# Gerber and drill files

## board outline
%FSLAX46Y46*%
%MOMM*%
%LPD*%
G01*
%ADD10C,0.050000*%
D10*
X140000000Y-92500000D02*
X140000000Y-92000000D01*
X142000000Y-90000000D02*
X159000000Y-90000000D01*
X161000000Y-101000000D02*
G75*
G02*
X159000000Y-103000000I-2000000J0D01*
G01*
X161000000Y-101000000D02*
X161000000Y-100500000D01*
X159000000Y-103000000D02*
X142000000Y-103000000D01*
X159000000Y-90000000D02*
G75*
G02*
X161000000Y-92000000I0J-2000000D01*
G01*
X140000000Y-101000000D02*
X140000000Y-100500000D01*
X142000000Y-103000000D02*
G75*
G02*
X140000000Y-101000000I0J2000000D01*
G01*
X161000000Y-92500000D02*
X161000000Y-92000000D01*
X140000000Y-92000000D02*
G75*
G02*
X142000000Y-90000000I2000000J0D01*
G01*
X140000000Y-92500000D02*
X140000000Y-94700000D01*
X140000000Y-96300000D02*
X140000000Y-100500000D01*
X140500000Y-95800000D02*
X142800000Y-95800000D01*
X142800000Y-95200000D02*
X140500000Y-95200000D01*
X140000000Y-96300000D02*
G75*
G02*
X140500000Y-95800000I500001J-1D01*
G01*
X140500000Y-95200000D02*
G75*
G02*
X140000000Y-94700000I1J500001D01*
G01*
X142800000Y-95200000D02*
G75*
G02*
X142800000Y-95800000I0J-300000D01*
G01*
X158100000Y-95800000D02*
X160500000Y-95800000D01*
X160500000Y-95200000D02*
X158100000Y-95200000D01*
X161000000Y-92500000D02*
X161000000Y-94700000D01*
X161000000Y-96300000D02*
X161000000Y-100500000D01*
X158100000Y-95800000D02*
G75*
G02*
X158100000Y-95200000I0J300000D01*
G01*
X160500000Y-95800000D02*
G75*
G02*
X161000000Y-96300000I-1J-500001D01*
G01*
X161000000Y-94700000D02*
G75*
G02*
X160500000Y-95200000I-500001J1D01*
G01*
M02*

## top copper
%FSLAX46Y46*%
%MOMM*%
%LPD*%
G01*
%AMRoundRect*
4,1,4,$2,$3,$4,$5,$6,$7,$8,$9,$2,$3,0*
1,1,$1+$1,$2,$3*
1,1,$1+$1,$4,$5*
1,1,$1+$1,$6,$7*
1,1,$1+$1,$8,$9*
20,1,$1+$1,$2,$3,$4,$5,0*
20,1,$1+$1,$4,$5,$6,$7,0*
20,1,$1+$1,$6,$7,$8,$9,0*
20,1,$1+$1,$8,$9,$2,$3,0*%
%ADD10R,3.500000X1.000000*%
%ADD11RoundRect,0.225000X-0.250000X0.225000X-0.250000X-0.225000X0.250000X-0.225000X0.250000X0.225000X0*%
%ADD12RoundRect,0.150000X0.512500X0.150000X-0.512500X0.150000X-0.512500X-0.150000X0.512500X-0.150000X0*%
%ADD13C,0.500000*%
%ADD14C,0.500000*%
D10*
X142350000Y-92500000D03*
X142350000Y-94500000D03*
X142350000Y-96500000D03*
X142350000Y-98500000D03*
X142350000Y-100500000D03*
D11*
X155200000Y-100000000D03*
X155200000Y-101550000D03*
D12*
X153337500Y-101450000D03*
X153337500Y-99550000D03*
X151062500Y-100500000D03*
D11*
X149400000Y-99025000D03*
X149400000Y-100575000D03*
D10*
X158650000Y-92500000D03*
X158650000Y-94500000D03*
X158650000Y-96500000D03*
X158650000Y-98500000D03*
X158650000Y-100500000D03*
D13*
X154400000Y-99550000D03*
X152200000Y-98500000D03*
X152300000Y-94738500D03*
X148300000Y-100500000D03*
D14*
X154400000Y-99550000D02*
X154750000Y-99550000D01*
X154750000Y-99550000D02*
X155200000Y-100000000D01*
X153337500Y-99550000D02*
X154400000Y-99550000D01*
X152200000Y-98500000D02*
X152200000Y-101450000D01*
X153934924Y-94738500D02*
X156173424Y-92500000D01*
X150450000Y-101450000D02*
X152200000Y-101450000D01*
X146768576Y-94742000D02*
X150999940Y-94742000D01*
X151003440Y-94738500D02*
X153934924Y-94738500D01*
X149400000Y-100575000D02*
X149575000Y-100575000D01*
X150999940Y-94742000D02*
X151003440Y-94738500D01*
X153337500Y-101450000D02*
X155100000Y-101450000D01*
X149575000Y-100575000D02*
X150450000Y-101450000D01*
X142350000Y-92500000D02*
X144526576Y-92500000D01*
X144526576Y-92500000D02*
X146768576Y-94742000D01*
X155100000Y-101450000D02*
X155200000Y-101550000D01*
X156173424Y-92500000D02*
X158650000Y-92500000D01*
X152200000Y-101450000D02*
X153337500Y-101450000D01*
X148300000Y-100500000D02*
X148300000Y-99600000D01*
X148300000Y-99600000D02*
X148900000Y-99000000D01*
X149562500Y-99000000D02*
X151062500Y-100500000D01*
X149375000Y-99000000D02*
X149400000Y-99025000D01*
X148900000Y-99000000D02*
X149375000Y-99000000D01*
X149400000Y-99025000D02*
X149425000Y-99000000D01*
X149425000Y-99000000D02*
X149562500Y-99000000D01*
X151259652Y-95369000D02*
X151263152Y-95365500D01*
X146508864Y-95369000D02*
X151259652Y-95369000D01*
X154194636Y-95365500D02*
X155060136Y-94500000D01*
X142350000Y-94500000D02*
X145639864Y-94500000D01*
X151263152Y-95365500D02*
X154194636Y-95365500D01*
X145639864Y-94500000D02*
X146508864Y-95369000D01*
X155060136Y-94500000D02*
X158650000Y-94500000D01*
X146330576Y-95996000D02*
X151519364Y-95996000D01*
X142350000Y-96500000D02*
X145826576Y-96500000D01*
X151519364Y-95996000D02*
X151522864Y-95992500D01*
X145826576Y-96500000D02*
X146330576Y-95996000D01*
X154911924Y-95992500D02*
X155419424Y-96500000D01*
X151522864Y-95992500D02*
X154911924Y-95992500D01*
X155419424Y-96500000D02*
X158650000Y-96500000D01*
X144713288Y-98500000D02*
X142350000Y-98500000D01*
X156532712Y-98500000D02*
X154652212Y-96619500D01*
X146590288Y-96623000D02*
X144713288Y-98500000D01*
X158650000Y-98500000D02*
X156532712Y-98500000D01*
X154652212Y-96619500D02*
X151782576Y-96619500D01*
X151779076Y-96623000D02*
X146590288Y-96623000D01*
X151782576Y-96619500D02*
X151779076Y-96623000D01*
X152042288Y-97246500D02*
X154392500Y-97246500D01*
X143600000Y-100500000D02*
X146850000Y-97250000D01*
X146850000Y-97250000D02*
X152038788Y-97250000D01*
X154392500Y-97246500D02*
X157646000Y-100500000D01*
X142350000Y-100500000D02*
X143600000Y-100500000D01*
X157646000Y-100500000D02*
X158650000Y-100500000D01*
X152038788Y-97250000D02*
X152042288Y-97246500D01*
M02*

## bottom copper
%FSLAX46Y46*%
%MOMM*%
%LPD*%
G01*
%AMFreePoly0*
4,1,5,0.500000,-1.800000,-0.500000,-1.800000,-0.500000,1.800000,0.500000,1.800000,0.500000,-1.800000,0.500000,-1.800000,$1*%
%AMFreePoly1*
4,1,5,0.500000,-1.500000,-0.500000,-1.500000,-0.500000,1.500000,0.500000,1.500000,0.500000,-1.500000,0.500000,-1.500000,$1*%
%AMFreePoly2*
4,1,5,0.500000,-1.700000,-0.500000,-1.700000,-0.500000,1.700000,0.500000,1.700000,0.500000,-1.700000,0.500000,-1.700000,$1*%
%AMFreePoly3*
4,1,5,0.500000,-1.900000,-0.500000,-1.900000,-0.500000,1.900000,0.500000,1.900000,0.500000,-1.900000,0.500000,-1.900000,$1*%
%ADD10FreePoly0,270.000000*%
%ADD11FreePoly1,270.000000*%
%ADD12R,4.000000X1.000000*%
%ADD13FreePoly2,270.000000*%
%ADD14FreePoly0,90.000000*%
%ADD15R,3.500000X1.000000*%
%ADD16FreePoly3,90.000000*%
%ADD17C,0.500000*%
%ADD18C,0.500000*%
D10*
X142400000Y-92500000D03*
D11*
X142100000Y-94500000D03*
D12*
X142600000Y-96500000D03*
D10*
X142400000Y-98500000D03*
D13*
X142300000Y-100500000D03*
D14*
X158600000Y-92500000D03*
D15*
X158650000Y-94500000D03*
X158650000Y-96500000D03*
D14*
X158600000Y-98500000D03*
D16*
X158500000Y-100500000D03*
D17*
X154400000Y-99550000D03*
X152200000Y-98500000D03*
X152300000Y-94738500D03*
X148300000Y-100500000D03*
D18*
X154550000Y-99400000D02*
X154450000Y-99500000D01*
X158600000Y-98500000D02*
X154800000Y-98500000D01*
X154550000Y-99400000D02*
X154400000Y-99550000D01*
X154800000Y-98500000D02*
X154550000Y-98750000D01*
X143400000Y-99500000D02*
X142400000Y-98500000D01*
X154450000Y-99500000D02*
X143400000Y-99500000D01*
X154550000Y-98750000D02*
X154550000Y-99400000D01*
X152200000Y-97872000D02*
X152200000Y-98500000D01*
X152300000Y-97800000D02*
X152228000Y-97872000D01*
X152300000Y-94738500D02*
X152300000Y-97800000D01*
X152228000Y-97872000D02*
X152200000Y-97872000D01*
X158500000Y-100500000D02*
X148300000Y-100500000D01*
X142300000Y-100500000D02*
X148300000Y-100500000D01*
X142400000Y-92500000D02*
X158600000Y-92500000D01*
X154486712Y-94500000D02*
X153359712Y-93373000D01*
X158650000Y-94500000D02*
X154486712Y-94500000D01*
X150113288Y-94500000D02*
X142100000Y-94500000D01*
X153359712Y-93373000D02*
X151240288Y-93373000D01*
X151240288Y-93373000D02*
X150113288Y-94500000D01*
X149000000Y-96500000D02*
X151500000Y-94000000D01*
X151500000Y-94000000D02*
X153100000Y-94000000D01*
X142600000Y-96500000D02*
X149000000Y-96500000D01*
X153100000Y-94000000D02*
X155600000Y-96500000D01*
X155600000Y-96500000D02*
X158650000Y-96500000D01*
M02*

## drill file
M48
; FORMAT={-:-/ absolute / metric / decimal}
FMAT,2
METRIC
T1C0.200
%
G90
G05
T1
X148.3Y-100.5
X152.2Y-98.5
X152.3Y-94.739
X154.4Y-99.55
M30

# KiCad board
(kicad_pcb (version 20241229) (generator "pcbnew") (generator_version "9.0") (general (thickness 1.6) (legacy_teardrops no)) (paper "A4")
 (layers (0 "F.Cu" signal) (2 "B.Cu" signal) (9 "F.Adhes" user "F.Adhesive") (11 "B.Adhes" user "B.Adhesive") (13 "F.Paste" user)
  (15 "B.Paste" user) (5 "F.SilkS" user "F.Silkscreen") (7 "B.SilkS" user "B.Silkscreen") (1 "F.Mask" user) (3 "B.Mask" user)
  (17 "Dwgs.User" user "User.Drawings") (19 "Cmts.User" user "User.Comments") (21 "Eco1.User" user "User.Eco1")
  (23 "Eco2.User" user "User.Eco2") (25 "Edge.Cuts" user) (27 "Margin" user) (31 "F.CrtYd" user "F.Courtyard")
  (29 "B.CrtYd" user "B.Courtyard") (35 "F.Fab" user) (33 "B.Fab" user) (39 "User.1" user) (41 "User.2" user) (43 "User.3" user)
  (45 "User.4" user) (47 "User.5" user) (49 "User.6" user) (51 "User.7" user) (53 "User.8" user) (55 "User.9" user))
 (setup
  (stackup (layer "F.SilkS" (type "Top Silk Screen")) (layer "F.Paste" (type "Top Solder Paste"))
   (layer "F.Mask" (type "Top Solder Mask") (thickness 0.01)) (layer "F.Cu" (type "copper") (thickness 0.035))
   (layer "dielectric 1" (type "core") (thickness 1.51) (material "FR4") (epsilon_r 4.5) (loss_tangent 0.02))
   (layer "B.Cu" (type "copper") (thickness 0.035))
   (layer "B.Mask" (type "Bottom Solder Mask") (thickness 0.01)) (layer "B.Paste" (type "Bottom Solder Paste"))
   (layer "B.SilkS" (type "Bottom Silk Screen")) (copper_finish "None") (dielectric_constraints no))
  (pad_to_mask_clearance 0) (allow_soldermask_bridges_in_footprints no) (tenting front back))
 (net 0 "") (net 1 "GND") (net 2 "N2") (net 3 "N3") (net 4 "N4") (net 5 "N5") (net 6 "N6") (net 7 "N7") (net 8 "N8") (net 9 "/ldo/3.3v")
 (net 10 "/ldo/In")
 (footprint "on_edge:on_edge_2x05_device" (layer "F.Cu") (at 140 96.5 -90)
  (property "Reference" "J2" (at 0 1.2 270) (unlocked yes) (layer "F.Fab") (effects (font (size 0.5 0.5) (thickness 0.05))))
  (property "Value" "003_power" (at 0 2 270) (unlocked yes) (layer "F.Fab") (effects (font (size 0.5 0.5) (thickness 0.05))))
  (fp_line (start -4 0) (end -1.8 0) (stroke (width 0.05) (type solid)) (layer "Edge.Cuts"))
  (fp_line (start -0.2 0) (end 4 0) (stroke (width 0.05) (type solid)) (layer "Edge.Cuts"))
  (fp_line (start -0.7 -0.5) (end -0.7 -2.8) (stroke (width 0.05) (type solid)) (layer "Edge.Cuts"))
  (fp_line (start -1.3 -2.8) (end -1.3 -0.5) (stroke (width 0.05) (type solid)) (layer "Edge.Cuts"))
  (fp_arc (start -0.2 0) (mid -0.553553 -0.146447) (end -0.7 -0.5) (stroke (width 0.05) (type solid)) (layer "Edge.Cuts"))
  (fp_arc (start -1.3 -0.5) (mid -1.446447 -0.146447) (end -1.8 0) (stroke (width 0.05) (type solid)) (layer "Edge.Cuts"))
  (fp_arc (start -1.3 -2.8) (mid -1 -3.1) (end -0.7 -2.8) (stroke (width 0.05) (type solid)) (layer "Edge.Cuts"))
  (pad "1" smd rect (at -4 -2.35 90) (size 1 3.5) (layers "F.Cu" "F.Mask") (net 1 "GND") (zone_connect 0))
  (pad "2" smd rect (at -2 -2.35 270) (size 1 3.5) (layers "F.Cu" "F.Mask") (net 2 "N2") (zone_connect 0))
  (pad "3" smd rect (at 0 -2.35 270) (size 1 3.5) (layers "F.Cu" "F.Mask") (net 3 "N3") (zone_connect 0))
  (pad "4" smd rect (at 2 -2.35 90) (size 1 3.5) (layers "F.Cu" "F.Mask") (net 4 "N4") (zone_connect 0))
  (pad "5" smd rect (at 4 -2.35 90) (size 1 3.5) (layers "F.Cu" "F.Mask") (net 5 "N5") (zone_connect 0))
  (pad "6" smd custom (at -4 -2.4 270) (size 1 3.6) (layers "B.Cu" "B.Mask") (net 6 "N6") (zone_connect 0)
   (options (clearance outline) (anchor rect)) (primitives))
  (pad "7" smd custom (at -2 -2.1 270) (size 1 3) (layers "B.Cu" "B.Mask") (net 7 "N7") (zone_connect 0)
   (options (clearance outline) (anchor rect)) (primitives))
  (pad "8" smd rect (at 0 -2.6 270) (size 1 4) (layers "B.Cu" "B.Mask") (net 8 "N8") (zone_connect 0))
  (pad "9" smd custom (at 2 -2.4 270) (size 1 3.6) (layers "B.Cu" "B.Mask") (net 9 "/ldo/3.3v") (zone_connect 0)
   (options (clearance outline) (anchor rect)) (primitives))
  (pad "10" smd custom (at 4 -2.3 270) (size 1 3.4) (layers "B.Cu" "B.Mask") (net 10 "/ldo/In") (zone_connect 0)
   (options (clearance outline) (anchor rect)) (primitives))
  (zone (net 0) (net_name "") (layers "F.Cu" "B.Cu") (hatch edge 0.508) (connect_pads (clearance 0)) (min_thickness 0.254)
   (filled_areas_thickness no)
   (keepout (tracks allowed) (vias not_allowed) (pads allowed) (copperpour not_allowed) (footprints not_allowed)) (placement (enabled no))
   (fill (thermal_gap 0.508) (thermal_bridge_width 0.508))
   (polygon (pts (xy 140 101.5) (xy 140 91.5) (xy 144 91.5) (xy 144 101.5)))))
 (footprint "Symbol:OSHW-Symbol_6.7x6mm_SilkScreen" (layer "F.Cu") (at 149.35 94.7)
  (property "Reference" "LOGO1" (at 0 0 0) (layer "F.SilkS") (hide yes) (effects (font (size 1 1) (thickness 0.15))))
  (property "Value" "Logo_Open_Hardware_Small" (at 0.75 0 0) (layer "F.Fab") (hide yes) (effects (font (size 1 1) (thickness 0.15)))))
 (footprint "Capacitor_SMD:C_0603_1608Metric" (layer "F.Cu") (at 155.2 100.775 -90)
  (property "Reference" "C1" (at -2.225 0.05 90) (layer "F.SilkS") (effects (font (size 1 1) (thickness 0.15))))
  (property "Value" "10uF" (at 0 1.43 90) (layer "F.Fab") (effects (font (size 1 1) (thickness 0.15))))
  (pad "1" smd roundrect (at -0.775 0 270) (size 0.9 0.95) (layers "F.Cu" "F.Mask" "F.Paste") (roundrect_rratio 0.25) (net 9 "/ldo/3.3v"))
  (pad "2" smd roundrect (at 0.775 0 270) (size 0.9 0.95) (layers "F.Cu" "F.Mask" "F.Paste") (roundrect_rratio 0.25) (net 1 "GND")))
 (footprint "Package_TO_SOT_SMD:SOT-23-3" (layer "F.Cu") (at 152.2 100.5 180)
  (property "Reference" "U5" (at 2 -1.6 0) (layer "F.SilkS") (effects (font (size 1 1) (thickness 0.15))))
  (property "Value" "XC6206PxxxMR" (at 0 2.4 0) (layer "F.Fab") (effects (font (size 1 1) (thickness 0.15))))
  (pad "1" smd roundrect (at -1.1375 -0.95 180) (size 1.325 0.6) (layers "F.Cu" "F.Mask" "F.Paste") (roundrect_rratio 0.25) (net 1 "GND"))
  (pad "2" smd roundrect (at -1.1375 0.95 180) (size 1.325 0.6) (layers "F.Cu" "F.Mask" "F.Paste") (roundrect_rratio 0.25)
   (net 9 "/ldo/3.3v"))
  (pad "3" smd roundrect (at 1.1375 0 180) (size 1.325 0.6) (layers "F.Cu" "F.Mask" "F.Paste") (roundrect_rratio 0.25) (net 10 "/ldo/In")))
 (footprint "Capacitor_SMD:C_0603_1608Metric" (layer "F.Cu") (at 149.4 99.8 -90)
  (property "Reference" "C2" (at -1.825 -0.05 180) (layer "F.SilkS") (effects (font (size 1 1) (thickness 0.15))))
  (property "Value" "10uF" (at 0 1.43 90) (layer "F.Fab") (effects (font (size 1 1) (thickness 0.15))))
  (pad "1" smd roundrect (at -0.775 0 270) (size 0.9 0.95) (layers "F.Cu" "F.Mask" "F.Paste") (roundrect_rratio 0.25) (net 10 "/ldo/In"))
  (pad "2" smd roundrect (at 0.775 0 270) (size 0.9 0.95) (layers "F.Cu" "F.Mask" "F.Paste") (roundrect_rratio 0.25) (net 1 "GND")))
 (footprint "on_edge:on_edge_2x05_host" (layer "F.Cu") (at 161 96.5 -90)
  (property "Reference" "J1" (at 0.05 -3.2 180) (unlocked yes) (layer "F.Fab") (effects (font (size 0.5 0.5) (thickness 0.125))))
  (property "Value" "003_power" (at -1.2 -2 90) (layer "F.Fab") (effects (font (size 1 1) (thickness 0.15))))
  (fp_line (start -0.7 2.9) (end -0.7 0.5) (stroke (width 0.05) (type solid)) (layer "Edge.Cuts"))
  (fp_line (start -1.3 0.5) (end -1.3 2.9) (stroke (width 0.05) (type solid)) (layer "Edge.Cuts"))
  (fp_line (start -4 0) (end -1.8 0) (stroke (width 0.05) (type solid)) (layer "Edge.Cuts"))
  (fp_line (start -0.2 0) (end 4 0) (stroke (width 0.05) (type solid)) (layer "Edge.Cuts"))
  (fp_arc (start -0.7 2.9) (mid -1 3.2) (end -1.3 2.9) (stroke (width 0.05) (type solid)) (layer "Edge.Cuts"))
  (fp_arc (start -0.7 0.5) (mid -0.553553 0.146447) (end -0.2 0) (stroke (width 0.05) (type solid)) (layer "Edge.Cuts"))
  (fp_arc (start -1.8 0) (mid -1.446447 0.146447) (end -1.3 0.5) (stroke (width 0.05) (type solid)) (layer "Edge.Cuts"))
  (pad "1" smd rect (at -4 2.35 270) (size 1 3.5) (layers "F.Cu" "F.Mask") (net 1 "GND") (zone_connect 0))
  (pad "2" smd rect (at -2 2.35 270) (size 1 3.5) (layers "F.Cu" "F.Mask") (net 2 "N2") (zone_connect 0))
  (pad "3" smd rect (at 0 2.35 270) (size 1 3.5) (layers "F.Cu" "F.Mask") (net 3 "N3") (zone_connect 0))
  (pad "4" smd rect (at 2 2.35 270) (size 1 3.5) (layers "F.Cu" "F.Mask") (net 4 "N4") (zone_connect 0))
  (pad "5" smd rect (at 4 2.35 270) (size 1 3.5) (layers "F.Cu" "F.Mask") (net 5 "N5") (zone_connect 0))
  (pad "6" smd custom (at -4 2.4 90) (size 1 3.6) (layers "B.Cu" "B.Mask") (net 6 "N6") (zone_connect 0)
   (options (clearance outline) (anchor rect)) (primitives))
  (pad "7" smd rect (at -2 2.35 90) (size 1 3.5) (layers "B.Cu" "B.Mask") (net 7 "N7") (zone_connect 0))
  (pad "8" smd rect (at 0 2.35 90) (size 1 3.5) (layers "B.Cu" "B.Mask") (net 8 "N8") (zone_connect 0))
  (pad "9" smd custom (at 2 2.4 90) (size 1 3.6) (layers "B.Cu" "B.Mask") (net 9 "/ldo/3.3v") (zone_connect 0)
   (options (clearance outline) (anchor rect)) (primitives))
  (pad "10" smd custom (at 4 2.5 90) (size 1 3.8) (layers "B.Cu" "B.Mask") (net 10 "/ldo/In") (zone_connect 0)
   (options (clearance outline) (anchor rect)) (primitives))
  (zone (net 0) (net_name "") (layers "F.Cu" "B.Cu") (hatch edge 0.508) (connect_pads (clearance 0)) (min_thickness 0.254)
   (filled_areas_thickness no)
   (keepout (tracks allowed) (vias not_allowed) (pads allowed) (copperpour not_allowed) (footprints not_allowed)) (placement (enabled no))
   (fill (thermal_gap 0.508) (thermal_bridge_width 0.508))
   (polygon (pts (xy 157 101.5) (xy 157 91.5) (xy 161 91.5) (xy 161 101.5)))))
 (gr_line (start 140 92.5) (end 140 92) (stroke (width 0.05) (type solid)) (layer "Edge.Cuts"))
 (gr_line (start 142 90) (end 159 90) (stroke (width 0.05) (type solid)) (layer "Edge.Cuts"))
 (gr_arc (start 161 101) (mid 160.414214 102.414214) (end 159 103) (stroke (width 0.05) (type solid)) (layer "Edge.Cuts"))
 (gr_line (start 161 101) (end 161 100.5) (stroke (width 0.05) (type solid)) (layer "Edge.Cuts"))
 (gr_line (start 159 103) (end 142 103) (stroke (width 0.05) (type solid)) (layer "Edge.Cuts"))
 (gr_arc (start 159 90) (mid 160.414214 90.585786) (end 161 92) (stroke (width 0.05) (type solid)) (layer "Edge.Cuts"))
 (gr_line (start 140 101) (end 140 100.5) (stroke (width 0.05) (type solid)) (layer "Edge.Cuts"))
 (gr_arc (start 142 103) (mid 140.585786 102.414214) (end 140 101) (stroke (width 0.05) (type solid)) (layer "Edge.Cuts"))
 (gr_line (start 161 92.5) (end 161 92) (stroke (width 0.05) (type solid)) (layer "Edge.Cuts"))
 (gr_arc (start 140 92) (mid 140.585786 90.585786) (end 142 90) (stroke (width 0.05) (type solid)) (layer "Edge.Cuts"))
 (segment (start 154.4 99.55) (end 154.75 99.55) (width 0.5) (layer "F.Cu") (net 9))
 (segment (start 154.75 99.55) (end 155.2 100) (width 0.5) (layer "F.Cu") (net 9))
 (segment (start 153.3375 99.55) (end 154.4 99.55) (width 0.5) (layer "F.Cu") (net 9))
 (via (at 154.4 99.55) (size 0.5) (drill 0.2) (layers "F.Cu" "B.Cu") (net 9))
 (segment (start 154.55 99.4) (end 154.45 99.5) (width 0.5) (layer "B.Cu") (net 9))
 (segment (start 158.6 98.5) (end 154.8 98.5) (width 0.5) (layer "B.Cu") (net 9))
 (segment (start 154.55 99.4) (end 154.4 99.55) (width 0.5) (layer "B.Cu") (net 9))
 (segment (start 154.8 98.5) (end 154.55 98.75) (width 0.5) (layer "B.Cu") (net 9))
 (segment (start 143.4 99.5) (end 142.4 98.5) (width 0.5) (layer "B.Cu") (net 9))
 (segment (start 154.45 99.5) (end 143.4 99.5) (width 0.5) (layer "B.Cu") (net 9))
 (segment (start 154.55 98.75) (end 154.55 99.4) (width 0.5) (layer "B.Cu") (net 9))
 (segment (start 152.2 98.5) (end 152.2 101.45) (width 0.5) (layer "F.Cu") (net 1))
 (segment (start 153.934924 94.7385) (end 156.173424 92.5) (width 0.5) (layer "F.Cu") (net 1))
 (segment (start 150.45 101.45) (end 152.2 101.45) (width 0.5) (layer "F.Cu") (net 1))
 (segment (start 146.768576 94.742) (end 150.99994 94.742) (width 0.5) (layer "F.Cu") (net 1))
 (segment (start 151.00344 94.7385) (end 153.934924 94.7385) (width 0.5) (layer "F.Cu") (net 1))
 (segment (start 149.4 100.575) (end 149.575 100.575) (width 0.5) (layer "F.Cu") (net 1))
 (segment (start 150.99994 94.742) (end 151.00344 94.7385) (width 0.5) (layer "F.Cu") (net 1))
 (segment (start 153.3375 101.45) (end 155.1 101.45) (width 0.5) (layer "F.Cu") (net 1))
 (segment (start 149.575 100.575) (end 150.45 101.45) (width 0.5) (layer "F.Cu") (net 1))
 (segment (start 142.35 92.5) (end 144.526576 92.5) (width 0.5) (layer "F.Cu") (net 1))
 (segment (start 144.526576 92.5) (end 146.768576 94.742) (width 0.5) (layer "F.Cu") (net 1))
 (segment (start 155.1 101.45) (end 155.2 101.55) (width 0.5) (layer "F.Cu") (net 1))
 (segment (start 156.173424 92.5) (end 158.65 92.5) (width 0.5) (layer "F.Cu") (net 1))
 (segment (start 152.2 101.45) (end 153.3375 101.45) (width 0.5) (layer "F.Cu") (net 1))
 (via (at 152.2 98.5) (size 0.5) (drill 0.2) (layers "F.Cu" "B.Cu") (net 1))
 (via (at 152.3 94.7385) (size 0.5) (drill 0.2) (layers "F.Cu" "B.Cu") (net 1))
 (segment (start 152.2 97.872) (end 152.2 98.5) (width 0.5) (layer "B.Cu") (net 1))
 (segment (start 152.3 97.8) (end 152.228 97.872) (width 0.5) (layer "B.Cu") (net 1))
 (segment (start 152.3 94.7385) (end 152.3 97.8) (width 0.5) (layer "B.Cu") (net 1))
 (segment (start 152.228 97.872) (end 152.2 97.872) (width 0.5) (layer "B.Cu") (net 1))
 (segment (start 148.3 100.5) (end 148.3 99.6) (width 0.5) (layer "F.Cu") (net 10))
 (segment (start 148.3 99.6) (end 148.9 99) (width 0.5) (layer "F.Cu") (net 10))
 (segment (start 149.5625 99) (end 151.0625 100.5) (width 0.5) (layer "F.Cu") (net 10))
 (segment (start 149.375 99) (end 149.4 99.025) (width 0.5) (layer "F.Cu") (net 10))
 (segment (start 148.9 99) (end 149.375 99) (width 0.5) (layer "F.Cu") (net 10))
 (segment (start 149.4 99.025) (end 149.425 99) (width 0.5) (layer "F.Cu") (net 10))
 (segment (start 149.425 99) (end 149.5625 99) (width 0.5) (layer "F.Cu") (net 10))
 (via (at 148.3 100.5) (size 0.5) (drill 0.2) (layers "F.Cu" "B.Cu") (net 10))
 (segment (start 158.5 100.5) (end 148.3 100.5) (width 0.5) (layer "B.Cu") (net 10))
 (segment (start 142.3 100.5) (end 148.3 100.5) (width 0.5) (layer "B.Cu") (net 10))
 (segment (start 151.259652 95.369) (end 151.263152 95.3655) (width 0.5) (layer "F.Cu") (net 2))
 (segment (start 146.508864 95.369) (end 151.259652 95.369) (width 0.5) (layer "F.Cu") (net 2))
 (segment (start 154.194636 95.3655) (end 155.060136 94.5) (width 0.5) (layer "F.Cu") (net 2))
 (segment (start 142.35 94.5) (end 145.639864 94.5) (width 0.5) (layer "F.Cu") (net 2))
 (segment (start 151.263152 95.3655) (end 154.194636 95.3655) (width 0.5) (layer "F.Cu") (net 2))
 (segment (start 145.639864 94.5) (end 146.508864 95.369) (width 0.5) (layer "F.Cu") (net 2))
 (segment (start 155.060136 94.5) (end 158.65 94.5) (width 0.5) (layer "F.Cu") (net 2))
 (segment (start 146.330576 95.996) (end 151.519364 95.996) (width 0.5) (layer "F.Cu") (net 3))
 (segment (start 142.35 96.5) (end 145.826576 96.5) (width 0.5) (layer "F.Cu") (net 3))
 (segment (start 151.519364 95.996) (end 151.522864 95.9925) (width 0.5) (layer "F.Cu") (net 3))
 (segment (start 145.826576 96.5) (end 146.330576 95.996) (width 0.5) (layer "F.Cu") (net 3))
 (segment (start 154.911924 95.9925) (end 155.419424 96.5) (width 0.5) (layer "F.Cu") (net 3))
 (segment (start 151.522864 95.9925) (end 154.911924 95.9925) (width 0.5) (layer "F.Cu") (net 3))
 (segment (start 155.419424 96.5) (end 158.65 96.5) (width 0.5) (layer "F.Cu") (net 3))
 (segment (start 144.713288 98.5) (end 142.35 98.5) (width 0.5) (layer "F.Cu") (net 4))
 (segment (start 156.532712 98.5) (end 154.652212 96.6195) (width 0.5) (layer "F.Cu") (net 4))
 (segment (start 146.590288 96.623) (end 144.713288 98.5) (width 0.5) (layer "F.Cu") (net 4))
 (segment (start 158.65 98.5) (end 156.532712 98.5) (width 0.5) (layer "F.Cu") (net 4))
 (segment (start 154.652212 96.6195) (end 151.782576 96.6195) (width 0.5) (layer "F.Cu") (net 4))
 (segment (start 151.779076 96.623) (end 146.590288 96.623) (width 0.5) (layer "F.Cu") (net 4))
 (segment (start 151.782576 96.6195) (end 151.779076 96.623) (width 0.5) (layer "F.Cu") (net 4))
 (segment (start 152.042288 97.2465) (end 154.3925 97.2465) (width 0.5) (layer "F.Cu") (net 5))
 (segment (start 143.6 100.5) (end 146.85 97.25) (width 0.5) (layer "F.Cu") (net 5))
 (segment (start 146.85 97.25) (end 152.038788 97.25) (width 0.5) (layer "F.Cu") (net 5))
 (segment (start 154.3925 97.2465) (end 157.646 100.5) (width 0.5) (layer "F.Cu") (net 5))
 (segment (start 142.35 100.5) (end 143.6 100.5) (width 0.5) (layer "F.Cu") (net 5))
 (segment (start 157.646 100.5) (end 158.65 100.5) (width 0.5) (layer "F.Cu") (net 5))
 (segment (start 152.038788 97.25) (end 152.042288 97.2465) (width 0.5) (layer "F.Cu") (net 5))
 (segment (start 142.4 92.5) (end 158.6 92.5) (width 0.5) (layer "B.Cu") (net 6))
 (segment (start 154.486712 94.5) (end 153.359712 93.373) (width 0.5) (layer "B.Cu") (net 7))
 (segment (start 158.65 94.5) (end 154.486712 94.5) (width 0.5) (layer "B.Cu") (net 7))
 (segment (start 150.113288 94.5) (end 142.1 94.5) (width 0.5) (layer "B.Cu") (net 7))
 (segment (start 153.359712 93.373) (end 151.240288 93.373) (width 0.5) (layer "B.Cu") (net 7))
 (segment (start 151.240288 93.373) (end 150.113288 94.5) (width 0.5) (layer "B.Cu") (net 7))
 (segment (start 149 96.5) (end 151.5 94) (width 0.5) (layer "B.Cu") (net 8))
 (segment (start 151.5 94) (end 153.1 94) (width 0.5) (layer "B.Cu") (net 8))
 (segment (start 142.6 96.5) (end 149 96.5) (width 0.5) (layer "B.Cu") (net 8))
 (segment (start 153.1 94) (end 155.6 96.5) (width 0.5) (layer "B.Cu") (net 8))
 (segment (start 155.6 96.5) (end 158.65 96.5) (width 0.5) (layer "B.Cu") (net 8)))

